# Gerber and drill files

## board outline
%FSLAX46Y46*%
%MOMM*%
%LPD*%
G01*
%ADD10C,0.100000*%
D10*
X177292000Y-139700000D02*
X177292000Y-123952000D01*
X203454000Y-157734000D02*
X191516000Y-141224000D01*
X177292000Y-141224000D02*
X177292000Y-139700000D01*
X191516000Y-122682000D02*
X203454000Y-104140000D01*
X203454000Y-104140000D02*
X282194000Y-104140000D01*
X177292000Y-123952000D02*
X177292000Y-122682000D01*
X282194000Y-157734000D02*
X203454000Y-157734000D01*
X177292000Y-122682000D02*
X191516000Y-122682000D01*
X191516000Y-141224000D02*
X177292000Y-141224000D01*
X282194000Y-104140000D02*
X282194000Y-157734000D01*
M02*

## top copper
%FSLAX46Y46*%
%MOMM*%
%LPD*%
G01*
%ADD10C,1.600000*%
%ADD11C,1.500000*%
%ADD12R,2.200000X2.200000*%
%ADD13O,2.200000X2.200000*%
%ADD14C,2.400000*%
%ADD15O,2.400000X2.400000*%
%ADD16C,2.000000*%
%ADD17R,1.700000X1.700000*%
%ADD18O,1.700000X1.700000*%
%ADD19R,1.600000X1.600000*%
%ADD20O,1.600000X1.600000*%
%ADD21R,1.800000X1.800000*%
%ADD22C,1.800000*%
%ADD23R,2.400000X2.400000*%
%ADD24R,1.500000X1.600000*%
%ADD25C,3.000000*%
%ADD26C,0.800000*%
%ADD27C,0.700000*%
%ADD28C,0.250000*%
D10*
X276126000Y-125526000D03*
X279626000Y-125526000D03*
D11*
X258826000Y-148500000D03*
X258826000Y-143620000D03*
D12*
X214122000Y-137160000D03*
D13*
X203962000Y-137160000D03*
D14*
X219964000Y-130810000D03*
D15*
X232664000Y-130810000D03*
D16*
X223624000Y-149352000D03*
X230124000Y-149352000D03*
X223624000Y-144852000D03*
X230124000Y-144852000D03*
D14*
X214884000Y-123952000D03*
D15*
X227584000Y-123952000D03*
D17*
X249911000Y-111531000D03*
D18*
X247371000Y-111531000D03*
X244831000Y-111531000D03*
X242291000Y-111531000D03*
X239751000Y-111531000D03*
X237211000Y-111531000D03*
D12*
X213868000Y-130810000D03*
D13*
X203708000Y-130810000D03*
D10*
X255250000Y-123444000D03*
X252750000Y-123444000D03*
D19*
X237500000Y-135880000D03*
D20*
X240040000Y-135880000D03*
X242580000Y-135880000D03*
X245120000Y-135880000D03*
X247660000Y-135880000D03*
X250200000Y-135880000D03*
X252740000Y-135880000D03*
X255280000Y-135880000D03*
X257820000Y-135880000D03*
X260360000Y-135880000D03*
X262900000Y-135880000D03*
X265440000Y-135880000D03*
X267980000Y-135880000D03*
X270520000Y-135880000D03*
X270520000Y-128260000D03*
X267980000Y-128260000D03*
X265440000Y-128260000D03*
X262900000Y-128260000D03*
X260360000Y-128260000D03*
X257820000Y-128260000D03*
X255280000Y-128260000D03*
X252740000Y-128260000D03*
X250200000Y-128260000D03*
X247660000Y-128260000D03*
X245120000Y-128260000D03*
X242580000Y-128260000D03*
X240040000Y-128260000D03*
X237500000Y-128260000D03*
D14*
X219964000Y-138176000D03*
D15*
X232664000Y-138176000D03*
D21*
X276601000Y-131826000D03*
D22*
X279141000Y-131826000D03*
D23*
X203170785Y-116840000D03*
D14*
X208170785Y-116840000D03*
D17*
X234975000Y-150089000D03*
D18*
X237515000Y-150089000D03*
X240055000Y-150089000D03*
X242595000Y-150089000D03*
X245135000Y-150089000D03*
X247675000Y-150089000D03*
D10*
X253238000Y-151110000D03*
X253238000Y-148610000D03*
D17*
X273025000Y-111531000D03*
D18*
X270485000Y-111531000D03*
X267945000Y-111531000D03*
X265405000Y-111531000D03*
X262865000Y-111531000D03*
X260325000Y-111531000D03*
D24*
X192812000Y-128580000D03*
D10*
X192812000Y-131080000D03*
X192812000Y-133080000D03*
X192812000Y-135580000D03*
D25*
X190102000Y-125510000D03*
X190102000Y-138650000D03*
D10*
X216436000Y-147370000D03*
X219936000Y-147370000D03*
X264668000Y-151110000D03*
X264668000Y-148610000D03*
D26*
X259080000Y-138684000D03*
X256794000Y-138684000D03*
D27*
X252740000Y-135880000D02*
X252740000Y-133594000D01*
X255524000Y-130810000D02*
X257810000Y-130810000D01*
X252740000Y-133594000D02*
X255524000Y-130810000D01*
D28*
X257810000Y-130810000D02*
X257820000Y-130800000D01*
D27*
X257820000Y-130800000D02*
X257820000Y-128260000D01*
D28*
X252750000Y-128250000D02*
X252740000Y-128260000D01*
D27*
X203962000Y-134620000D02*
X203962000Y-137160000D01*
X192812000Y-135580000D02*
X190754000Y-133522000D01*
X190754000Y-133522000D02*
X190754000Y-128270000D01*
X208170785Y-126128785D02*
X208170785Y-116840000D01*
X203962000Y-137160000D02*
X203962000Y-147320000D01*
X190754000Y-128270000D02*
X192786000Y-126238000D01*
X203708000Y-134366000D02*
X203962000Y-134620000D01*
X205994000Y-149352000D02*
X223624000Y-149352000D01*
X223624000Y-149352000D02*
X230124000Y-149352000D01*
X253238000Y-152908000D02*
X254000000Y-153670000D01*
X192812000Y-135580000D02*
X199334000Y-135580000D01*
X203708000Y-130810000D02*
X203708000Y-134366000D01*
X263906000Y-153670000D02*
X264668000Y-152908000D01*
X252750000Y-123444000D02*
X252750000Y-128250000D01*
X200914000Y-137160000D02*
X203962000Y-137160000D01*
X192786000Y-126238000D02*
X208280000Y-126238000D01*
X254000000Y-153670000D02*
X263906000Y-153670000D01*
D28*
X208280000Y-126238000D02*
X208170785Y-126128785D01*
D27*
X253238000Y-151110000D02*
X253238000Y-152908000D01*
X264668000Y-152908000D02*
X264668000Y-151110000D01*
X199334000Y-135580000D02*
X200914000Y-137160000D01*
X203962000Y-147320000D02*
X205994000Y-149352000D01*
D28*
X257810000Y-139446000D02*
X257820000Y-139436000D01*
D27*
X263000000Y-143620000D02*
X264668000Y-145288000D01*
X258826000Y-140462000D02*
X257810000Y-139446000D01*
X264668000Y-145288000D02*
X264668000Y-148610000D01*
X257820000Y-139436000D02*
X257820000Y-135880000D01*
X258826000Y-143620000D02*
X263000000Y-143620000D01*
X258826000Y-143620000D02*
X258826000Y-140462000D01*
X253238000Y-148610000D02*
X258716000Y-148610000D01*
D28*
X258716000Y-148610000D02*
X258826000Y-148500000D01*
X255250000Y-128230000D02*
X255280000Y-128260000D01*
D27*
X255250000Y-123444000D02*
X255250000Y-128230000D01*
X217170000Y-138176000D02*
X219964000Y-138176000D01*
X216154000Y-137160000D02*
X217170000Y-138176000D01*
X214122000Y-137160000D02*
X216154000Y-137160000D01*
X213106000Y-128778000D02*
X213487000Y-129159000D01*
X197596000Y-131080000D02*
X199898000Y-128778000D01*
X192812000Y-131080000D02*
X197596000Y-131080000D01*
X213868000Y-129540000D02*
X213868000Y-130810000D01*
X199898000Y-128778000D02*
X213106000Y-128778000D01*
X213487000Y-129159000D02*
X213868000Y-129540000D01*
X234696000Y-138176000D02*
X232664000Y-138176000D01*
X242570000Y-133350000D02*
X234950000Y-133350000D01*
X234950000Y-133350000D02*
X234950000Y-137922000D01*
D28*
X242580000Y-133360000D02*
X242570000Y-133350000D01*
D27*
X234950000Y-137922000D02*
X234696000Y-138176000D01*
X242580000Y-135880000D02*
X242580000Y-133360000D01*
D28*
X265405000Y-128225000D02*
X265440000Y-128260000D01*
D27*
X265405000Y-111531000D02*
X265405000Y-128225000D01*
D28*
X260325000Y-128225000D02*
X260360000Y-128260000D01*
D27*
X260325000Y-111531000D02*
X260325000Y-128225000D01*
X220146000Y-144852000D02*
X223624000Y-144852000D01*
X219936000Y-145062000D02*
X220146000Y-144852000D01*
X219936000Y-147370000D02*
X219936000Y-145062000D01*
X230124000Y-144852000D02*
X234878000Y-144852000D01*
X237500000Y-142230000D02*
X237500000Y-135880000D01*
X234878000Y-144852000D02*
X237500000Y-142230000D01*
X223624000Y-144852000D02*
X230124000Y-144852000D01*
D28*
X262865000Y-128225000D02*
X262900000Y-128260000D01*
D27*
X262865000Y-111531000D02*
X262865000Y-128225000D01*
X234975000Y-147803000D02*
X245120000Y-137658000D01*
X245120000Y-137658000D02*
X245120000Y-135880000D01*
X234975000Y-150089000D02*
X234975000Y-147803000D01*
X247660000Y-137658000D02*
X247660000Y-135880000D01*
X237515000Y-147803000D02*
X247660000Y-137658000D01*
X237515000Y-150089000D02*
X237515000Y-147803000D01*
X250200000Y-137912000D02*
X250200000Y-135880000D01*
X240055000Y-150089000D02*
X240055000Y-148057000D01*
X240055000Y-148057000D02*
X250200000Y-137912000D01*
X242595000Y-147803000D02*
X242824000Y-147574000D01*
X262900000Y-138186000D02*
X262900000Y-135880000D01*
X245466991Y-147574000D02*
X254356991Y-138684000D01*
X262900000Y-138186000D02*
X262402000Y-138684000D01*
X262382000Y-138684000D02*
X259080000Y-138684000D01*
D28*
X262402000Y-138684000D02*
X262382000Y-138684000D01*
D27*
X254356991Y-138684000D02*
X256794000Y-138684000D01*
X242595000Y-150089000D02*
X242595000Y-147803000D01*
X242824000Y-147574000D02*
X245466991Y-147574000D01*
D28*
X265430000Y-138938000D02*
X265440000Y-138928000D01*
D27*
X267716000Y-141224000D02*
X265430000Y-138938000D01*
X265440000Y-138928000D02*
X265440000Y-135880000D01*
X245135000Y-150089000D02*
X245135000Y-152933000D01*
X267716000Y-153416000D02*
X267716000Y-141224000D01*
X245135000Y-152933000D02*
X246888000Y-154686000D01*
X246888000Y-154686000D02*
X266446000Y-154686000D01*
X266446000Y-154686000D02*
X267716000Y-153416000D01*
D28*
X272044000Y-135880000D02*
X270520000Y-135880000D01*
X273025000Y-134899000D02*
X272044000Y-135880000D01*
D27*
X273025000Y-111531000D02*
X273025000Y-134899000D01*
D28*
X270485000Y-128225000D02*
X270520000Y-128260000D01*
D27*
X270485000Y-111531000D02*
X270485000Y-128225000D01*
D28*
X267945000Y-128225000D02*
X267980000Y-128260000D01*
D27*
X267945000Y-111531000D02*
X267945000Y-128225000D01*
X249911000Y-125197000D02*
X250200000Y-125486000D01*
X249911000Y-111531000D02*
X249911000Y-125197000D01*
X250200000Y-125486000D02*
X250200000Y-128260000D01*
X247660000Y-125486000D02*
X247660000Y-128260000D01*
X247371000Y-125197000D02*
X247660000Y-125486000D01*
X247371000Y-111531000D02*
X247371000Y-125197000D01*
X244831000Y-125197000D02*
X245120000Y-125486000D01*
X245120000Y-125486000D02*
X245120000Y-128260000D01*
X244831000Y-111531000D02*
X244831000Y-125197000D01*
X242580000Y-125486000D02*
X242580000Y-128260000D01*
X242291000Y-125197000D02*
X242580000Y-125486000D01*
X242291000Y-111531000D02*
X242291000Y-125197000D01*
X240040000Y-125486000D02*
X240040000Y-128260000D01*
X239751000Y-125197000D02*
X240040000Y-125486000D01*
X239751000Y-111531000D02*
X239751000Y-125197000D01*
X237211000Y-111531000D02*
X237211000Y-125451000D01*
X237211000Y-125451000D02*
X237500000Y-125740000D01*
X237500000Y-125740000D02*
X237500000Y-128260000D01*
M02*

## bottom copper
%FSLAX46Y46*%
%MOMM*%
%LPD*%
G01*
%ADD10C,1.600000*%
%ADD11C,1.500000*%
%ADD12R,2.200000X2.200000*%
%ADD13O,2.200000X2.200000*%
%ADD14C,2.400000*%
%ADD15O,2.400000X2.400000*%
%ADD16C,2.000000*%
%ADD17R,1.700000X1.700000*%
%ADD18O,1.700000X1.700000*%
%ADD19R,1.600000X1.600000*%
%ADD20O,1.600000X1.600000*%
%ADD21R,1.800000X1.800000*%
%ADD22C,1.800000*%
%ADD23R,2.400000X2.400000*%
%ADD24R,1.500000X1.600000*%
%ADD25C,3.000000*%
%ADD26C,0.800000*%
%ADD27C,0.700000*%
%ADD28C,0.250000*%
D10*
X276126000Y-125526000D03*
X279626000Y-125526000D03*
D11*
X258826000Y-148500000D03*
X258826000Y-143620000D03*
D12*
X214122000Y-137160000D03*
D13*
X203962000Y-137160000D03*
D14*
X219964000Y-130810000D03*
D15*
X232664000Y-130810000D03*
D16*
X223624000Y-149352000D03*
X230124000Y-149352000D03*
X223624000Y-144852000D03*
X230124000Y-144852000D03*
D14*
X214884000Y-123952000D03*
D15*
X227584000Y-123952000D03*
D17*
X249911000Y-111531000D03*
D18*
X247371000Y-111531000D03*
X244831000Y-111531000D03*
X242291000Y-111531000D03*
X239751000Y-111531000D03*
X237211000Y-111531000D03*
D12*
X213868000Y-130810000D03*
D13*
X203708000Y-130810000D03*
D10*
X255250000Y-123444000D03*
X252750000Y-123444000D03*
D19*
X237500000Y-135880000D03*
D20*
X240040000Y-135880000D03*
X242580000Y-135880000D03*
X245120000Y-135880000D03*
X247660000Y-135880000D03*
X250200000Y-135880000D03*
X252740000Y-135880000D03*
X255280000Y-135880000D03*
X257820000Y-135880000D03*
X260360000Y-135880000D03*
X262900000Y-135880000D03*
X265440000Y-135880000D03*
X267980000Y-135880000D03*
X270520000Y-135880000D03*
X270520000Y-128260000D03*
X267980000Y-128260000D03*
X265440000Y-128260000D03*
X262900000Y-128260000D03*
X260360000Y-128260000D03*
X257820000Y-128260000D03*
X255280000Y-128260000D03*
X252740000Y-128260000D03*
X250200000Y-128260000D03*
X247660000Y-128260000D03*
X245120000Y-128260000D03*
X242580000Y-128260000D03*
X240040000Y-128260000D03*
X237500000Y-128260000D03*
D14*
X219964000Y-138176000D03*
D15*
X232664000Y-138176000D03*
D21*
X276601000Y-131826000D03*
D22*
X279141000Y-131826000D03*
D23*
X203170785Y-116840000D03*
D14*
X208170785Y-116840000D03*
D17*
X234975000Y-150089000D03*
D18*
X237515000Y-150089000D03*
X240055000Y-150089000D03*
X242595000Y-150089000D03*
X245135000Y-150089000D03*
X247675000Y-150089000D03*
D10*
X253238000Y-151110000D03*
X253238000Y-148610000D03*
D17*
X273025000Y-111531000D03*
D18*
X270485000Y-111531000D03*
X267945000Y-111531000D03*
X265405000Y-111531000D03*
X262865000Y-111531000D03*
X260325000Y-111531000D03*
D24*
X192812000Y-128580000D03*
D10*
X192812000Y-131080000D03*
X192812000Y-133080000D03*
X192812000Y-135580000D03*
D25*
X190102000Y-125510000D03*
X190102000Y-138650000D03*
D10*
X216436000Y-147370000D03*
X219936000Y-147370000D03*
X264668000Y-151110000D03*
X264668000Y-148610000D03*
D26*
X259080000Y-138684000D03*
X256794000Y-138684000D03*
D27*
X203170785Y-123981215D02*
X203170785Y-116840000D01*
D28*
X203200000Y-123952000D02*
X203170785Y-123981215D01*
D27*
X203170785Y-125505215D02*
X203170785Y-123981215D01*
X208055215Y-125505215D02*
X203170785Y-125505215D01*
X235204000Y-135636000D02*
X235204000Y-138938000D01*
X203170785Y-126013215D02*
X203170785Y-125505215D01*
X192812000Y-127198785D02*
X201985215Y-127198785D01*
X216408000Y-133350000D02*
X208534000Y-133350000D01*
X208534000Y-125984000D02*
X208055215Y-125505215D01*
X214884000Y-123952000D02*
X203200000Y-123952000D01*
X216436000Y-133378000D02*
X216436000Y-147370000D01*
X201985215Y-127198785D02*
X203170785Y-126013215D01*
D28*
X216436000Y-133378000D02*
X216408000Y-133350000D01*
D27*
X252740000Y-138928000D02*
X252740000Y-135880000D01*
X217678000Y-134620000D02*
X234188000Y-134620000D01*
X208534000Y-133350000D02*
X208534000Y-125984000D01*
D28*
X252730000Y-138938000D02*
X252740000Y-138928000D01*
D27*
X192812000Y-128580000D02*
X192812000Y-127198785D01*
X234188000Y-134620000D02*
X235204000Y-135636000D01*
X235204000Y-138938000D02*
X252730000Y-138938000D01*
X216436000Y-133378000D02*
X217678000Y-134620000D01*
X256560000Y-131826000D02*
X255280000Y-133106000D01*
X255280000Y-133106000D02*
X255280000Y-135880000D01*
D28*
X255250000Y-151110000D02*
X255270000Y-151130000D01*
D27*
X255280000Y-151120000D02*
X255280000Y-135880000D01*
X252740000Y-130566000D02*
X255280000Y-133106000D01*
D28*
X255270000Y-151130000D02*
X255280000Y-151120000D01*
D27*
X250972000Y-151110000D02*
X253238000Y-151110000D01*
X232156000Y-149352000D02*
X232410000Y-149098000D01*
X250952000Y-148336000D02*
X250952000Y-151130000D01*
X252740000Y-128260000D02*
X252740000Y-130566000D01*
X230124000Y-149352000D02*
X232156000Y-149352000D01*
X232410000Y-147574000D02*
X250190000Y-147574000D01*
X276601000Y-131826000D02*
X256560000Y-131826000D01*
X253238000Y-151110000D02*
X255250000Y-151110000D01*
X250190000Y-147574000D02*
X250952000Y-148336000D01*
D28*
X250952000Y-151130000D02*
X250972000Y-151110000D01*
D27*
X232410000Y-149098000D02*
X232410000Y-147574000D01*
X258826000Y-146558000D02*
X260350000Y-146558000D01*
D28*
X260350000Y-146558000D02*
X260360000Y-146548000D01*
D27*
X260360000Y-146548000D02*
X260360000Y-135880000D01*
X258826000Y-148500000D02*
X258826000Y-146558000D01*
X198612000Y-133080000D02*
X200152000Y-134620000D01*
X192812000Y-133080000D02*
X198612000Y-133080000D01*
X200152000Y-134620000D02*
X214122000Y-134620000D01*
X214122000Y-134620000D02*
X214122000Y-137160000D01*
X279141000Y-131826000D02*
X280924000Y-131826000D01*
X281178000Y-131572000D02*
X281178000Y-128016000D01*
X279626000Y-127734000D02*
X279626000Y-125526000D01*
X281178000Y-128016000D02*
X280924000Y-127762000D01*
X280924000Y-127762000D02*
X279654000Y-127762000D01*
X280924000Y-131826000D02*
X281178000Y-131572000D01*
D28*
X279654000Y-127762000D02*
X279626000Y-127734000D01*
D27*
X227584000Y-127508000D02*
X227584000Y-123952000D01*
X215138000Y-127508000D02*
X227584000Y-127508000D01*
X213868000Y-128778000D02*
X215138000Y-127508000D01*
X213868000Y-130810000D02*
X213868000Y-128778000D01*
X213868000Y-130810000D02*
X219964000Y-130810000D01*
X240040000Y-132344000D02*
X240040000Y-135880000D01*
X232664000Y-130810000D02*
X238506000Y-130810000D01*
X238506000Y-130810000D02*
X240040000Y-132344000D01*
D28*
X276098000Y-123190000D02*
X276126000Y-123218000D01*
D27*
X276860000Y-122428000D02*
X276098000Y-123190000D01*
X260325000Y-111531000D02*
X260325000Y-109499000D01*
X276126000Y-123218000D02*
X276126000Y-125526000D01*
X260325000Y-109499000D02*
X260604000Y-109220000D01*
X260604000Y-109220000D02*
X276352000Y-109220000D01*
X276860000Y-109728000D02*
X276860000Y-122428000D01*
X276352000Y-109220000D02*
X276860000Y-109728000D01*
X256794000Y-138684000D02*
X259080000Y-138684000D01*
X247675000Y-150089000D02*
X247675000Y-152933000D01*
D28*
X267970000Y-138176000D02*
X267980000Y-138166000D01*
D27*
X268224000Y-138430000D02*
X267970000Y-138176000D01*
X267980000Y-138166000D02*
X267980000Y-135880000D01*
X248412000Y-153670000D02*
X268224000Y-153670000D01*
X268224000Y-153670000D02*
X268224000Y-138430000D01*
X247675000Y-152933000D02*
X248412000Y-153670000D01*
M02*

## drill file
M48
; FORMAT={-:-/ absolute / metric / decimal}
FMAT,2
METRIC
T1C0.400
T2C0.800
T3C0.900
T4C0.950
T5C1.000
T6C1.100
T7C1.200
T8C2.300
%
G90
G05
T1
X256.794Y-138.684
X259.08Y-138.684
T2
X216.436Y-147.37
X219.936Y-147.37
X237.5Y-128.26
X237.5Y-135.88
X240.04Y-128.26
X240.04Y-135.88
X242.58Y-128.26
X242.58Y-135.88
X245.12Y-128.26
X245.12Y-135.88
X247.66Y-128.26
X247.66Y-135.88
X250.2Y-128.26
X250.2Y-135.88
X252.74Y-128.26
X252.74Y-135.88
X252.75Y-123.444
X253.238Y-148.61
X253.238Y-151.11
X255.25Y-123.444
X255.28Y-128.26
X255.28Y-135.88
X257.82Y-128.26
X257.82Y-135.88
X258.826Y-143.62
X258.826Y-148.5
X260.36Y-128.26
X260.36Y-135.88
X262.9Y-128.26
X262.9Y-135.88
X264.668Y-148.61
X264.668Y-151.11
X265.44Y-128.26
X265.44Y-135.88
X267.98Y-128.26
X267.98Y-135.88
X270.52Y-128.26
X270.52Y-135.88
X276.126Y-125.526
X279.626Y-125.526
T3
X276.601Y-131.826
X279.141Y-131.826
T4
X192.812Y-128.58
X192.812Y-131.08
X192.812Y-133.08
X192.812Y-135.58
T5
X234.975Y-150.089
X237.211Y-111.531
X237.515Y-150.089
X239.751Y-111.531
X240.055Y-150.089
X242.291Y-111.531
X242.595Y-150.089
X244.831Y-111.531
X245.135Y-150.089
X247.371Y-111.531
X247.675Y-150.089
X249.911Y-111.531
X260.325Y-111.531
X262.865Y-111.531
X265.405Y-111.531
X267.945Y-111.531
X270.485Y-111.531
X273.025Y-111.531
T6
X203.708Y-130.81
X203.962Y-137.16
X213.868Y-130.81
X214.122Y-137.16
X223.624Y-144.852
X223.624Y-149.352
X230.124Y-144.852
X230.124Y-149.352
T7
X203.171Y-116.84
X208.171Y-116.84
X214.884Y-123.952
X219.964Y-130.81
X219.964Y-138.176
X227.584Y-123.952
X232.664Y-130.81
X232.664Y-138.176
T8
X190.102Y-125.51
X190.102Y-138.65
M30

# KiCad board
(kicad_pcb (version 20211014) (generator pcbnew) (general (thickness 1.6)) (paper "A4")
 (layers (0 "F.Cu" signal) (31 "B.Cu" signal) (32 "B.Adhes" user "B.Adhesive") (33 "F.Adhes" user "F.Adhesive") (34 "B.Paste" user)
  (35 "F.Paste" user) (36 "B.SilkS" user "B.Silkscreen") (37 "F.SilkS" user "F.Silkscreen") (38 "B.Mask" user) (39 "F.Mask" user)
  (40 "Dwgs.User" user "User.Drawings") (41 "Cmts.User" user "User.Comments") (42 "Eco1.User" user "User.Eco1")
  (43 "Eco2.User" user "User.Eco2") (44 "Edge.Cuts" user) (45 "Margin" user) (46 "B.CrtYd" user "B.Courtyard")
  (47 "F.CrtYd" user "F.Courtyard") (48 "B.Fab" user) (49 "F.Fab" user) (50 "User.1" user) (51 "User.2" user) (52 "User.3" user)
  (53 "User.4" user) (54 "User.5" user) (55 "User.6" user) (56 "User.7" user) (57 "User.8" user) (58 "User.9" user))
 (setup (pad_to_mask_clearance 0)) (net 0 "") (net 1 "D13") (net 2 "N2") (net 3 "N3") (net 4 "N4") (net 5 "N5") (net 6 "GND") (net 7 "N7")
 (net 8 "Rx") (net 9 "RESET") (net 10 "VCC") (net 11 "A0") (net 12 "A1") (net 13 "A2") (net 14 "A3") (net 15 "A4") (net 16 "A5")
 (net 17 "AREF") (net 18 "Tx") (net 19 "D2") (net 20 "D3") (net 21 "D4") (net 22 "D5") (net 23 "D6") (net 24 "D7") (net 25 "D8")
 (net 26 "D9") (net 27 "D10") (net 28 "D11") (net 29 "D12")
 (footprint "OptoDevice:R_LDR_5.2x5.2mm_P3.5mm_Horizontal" (layer "F.Cu") (at 276.126 125.526)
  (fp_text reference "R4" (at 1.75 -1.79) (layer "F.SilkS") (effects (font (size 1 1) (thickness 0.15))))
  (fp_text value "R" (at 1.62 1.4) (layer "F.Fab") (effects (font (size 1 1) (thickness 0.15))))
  (pad "1" thru_hole circle (at 0 0) (size 1.6 1.6) (drill 0.8) (layers *.Cu *.Mask) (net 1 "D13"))
  (pad "2" thru_hole circle (at 3.5 0) (size 1.6 1.6) (drill 0.8) (layers *.Cu *.Mask) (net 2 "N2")))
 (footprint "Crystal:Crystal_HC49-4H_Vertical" (layer "F.Cu") (at 258.826 148.5 90)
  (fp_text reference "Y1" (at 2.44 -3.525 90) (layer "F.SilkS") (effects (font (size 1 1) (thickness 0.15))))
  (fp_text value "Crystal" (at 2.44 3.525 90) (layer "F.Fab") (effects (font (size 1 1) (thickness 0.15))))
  (pad "1" thru_hole circle (at 0 0 90) (size 1.5 1.5) (drill 0.8) (layers *.Cu *.Mask) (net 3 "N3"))
  (pad "2" thru_hole circle (at 4.88 0 90) (size 1.5 1.5) (drill 0.8) (layers *.Cu *.Mask) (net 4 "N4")))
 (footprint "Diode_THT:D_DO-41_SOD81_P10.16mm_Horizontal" (layer "F.Cu") (at 214.122 137.16 180)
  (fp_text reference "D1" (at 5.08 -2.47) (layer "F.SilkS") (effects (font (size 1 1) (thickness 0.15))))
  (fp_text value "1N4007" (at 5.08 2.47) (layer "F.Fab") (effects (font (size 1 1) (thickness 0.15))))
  (pad "1" thru_hole rect (at 0 0 180) (size 2.2 2.2) (drill 1.1) (layers *.Cu *.Mask) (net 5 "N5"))
  (pad "2" thru_hole oval (at 10.16 0 180) (size 2.2 2.2) (drill 1.1) (layers *.Cu *.Mask) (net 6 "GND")))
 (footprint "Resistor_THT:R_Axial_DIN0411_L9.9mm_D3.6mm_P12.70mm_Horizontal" (layer "F.Cu") (at 219.964 130.81)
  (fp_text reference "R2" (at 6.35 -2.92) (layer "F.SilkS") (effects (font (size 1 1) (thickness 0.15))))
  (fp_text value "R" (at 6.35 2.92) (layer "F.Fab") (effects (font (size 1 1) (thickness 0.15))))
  (pad "1" thru_hole circle (at 0 0) (size 2.4 2.4) (drill 1.2) (layers *.Cu *.Mask) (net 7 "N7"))
  (pad "2" thru_hole oval (at 12.7 0) (size 2.4 2.4) (drill 1.2) (layers *.Cu *.Mask) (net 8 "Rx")))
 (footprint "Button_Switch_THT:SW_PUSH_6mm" (layer "F.Cu") (at 230.124 149.352 180)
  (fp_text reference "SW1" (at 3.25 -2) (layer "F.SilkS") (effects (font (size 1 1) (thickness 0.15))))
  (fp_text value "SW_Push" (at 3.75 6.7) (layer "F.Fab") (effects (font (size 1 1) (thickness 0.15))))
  (pad "1" thru_hole circle (at 6.5 0 270) (size 2 2) (drill 1.1) (layers *.Cu *.Mask) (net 6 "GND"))
  (pad "1" thru_hole circle (at 0 0 270) (size 2 2) (drill 1.1) (layers *.Cu *.Mask) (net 6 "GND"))
  (pad "2" thru_hole circle (at 6.5 4.5 270) (size 2 2) (drill 1.1) (layers *.Cu *.Mask) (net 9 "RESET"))
  (pad "2" thru_hole circle (at 0 4.5 270) (size 2 2) (drill 1.1) (layers *.Cu *.Mask) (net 9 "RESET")))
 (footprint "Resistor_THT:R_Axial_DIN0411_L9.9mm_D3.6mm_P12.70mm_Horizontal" (layer "F.Cu") (at 214.884 123.952)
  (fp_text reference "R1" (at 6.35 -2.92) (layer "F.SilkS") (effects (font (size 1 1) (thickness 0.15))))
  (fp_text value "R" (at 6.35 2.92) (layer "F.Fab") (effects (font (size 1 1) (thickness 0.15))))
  (pad "1" thru_hole circle (at 0 0) (size 2.4 2.4) (drill 1.2) (layers *.Cu *.Mask) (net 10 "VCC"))
  (pad "2" thru_hole oval (at 12.7 0) (size 2.4 2.4) (drill 1.2) (layers *.Cu *.Mask) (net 7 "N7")))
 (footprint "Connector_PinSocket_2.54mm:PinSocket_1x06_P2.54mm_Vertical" (layer "F.Cu") (at 249.911 111.531 -90)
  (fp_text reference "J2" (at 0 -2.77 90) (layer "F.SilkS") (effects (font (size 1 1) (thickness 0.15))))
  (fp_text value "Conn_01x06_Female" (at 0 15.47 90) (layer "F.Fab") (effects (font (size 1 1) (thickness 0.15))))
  (pad "1" thru_hole rect (at 0 0 270) (size 1.7 1.7) (drill 1) (layers *.Cu *.Mask) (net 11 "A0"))
  (pad "2" thru_hole oval (at 0 2.54 270) (size 1.7 1.7) (drill 1) (layers *.Cu *.Mask) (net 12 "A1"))
  (pad "3" thru_hole oval (at 0 5.08 270) (size 1.7 1.7) (drill 1) (layers *.Cu *.Mask) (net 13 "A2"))
  (pad "4" thru_hole oval (at 0 7.62 270) (size 1.7 1.7) (drill 1) (layers *.Cu *.Mask) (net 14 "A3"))
  (pad "5" thru_hole oval (at 0 10.16 270) (size 1.7 1.7) (drill 1) (layers *.Cu *.Mask) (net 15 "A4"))
  (pad "6" thru_hole oval (at 0 12.7 270) (size 1.7 1.7) (drill 1) (layers *.Cu *.Mask) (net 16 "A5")))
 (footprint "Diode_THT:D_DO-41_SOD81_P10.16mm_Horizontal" (layer "F.Cu") (at 213.868 130.81 180)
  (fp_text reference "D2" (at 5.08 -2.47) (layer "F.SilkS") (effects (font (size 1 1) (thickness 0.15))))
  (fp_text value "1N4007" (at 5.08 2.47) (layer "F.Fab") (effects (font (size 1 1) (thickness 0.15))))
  (pad "1" thru_hole rect (at 0 0 180) (size 2.2 2.2) (drill 1.1) (layers *.Cu *.Mask) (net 7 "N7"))
  (pad "2" thru_hole oval (at 10.16 0 180) (size 2.2 2.2) (drill 1.1) (layers *.Cu *.Mask) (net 6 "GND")))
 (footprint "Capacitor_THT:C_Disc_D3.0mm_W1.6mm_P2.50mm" (layer "F.Cu") (at 255.25 123.444 180)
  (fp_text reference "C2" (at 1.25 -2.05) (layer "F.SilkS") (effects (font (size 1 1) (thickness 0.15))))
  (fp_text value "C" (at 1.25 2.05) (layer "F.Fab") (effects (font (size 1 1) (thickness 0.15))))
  (pad "1" thru_hole circle (at 0 0 180) (size 1.6 1.6) (drill 0.8) (layers *.Cu *.Mask) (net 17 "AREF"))
  (pad "2" thru_hole circle (at 2.5 0 180) (size 1.6 1.6) (drill 0.8) (layers *.Cu *.Mask) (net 6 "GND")))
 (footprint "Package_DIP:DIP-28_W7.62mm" (layer "F.Cu") (at 237.5 135.88 90)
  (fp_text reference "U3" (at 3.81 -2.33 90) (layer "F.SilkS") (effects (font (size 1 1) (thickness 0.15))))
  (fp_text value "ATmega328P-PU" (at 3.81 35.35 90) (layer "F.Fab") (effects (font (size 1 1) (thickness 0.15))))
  (pad "1" thru_hole rect (at 0 0 90) (size 1.6 1.6) (drill 0.8) (layers *.Cu *.Mask) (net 9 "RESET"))
  (pad "2" thru_hole oval (at 0 2.54 90) (size 1.6 1.6) (drill 0.8) (layers *.Cu *.Mask) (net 8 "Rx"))
  (pad "3" thru_hole oval (at 0 5.08 90) (size 1.6 1.6) (drill 0.8) (layers *.Cu *.Mask) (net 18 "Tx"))
  (pad "4" thru_hole oval (at 0 7.62 90) (size 1.6 1.6) (drill 0.8) (layers *.Cu *.Mask) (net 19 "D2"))
  (pad "5" thru_hole oval (at 0 10.16 90) (size 1.6 1.6) (drill 0.8) (layers *.Cu *.Mask) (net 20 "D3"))
  (pad "6" thru_hole oval (at 0 12.7 90) (size 1.6 1.6) (drill 0.8) (layers *.Cu *.Mask) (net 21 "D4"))
  (pad "7" thru_hole oval (at 0 15.24 90) (size 1.6 1.6) (drill 0.8) (layers *.Cu *.Mask) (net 10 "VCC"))
  (pad "8" thru_hole oval (at 0 17.78 90) (size 1.6 1.6) (drill 0.8) (layers *.Cu *.Mask) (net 6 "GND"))
  (pad "9" thru_hole oval (at 0 20.32 90) (size 1.6 1.6) (drill 0.8) (layers *.Cu *.Mask) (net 4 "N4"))
  (pad "10" thru_hole oval (at 0 22.86 90) (size 1.6 1.6) (drill 0.8) (layers *.Cu *.Mask) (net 3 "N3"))
  (pad "11" thru_hole oval (at 0 25.4 90) (size 1.6 1.6) (drill 0.8) (layers *.Cu *.Mask) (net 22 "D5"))
  (pad "12" thru_hole oval (at 0 27.94 90) (size 1.6 1.6) (drill 0.8) (layers *.Cu *.Mask) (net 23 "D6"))
  (pad "13" thru_hole oval (at 0 30.48 90) (size 1.6 1.6) (drill 0.8) (layers *.Cu *.Mask) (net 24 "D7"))
  (pad "14" thru_hole oval (at 0 33.02 90) (size 1.6 1.6) (drill 0.8) (layers *.Cu *.Mask) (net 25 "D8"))
  (pad "15" thru_hole oval (at 7.62 33.02 90) (size 1.6 1.6) (drill 0.8) (layers *.Cu *.Mask) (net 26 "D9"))
  (pad "16" thru_hole oval (at 7.62 30.48 90) (size 1.6 1.6) (drill 0.8) (layers *.Cu *.Mask) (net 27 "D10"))
  (pad "17" thru_hole oval (at 7.62 27.94 90) (size 1.6 1.6) (drill 0.8) (layers *.Cu *.Mask) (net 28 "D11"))
  (pad "18" thru_hole oval (at 7.62 25.4 90) (size 1.6 1.6) (drill 0.8) (layers *.Cu *.Mask) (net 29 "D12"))
  (pad "19" thru_hole oval (at 7.62 22.86 90) (size 1.6 1.6) (drill 0.8) (layers *.Cu *.Mask) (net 1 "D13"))
  (pad "20" thru_hole oval (at 7.62 20.32 90) (size 1.6 1.6) (drill 0.8) (layers *.Cu *.Mask) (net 10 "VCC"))
  (pad "21" thru_hole oval (at 7.62 17.78 90) (size 1.6 1.6) (drill 0.8) (layers *.Cu *.Mask) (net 17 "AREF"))
  (pad "22" thru_hole oval (at 7.62 15.24 90) (size 1.6 1.6) (drill 0.8) (layers *.Cu *.Mask) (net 6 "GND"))
  (pad "23" thru_hole oval (at 7.62 12.7 90) (size 1.6 1.6) (drill 0.8) (layers *.Cu *.Mask) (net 11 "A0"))
  (pad "24" thru_hole oval (at 7.62 10.16 90) (size 1.6 1.6) (drill 0.8) (layers *.Cu *.Mask) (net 12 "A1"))
  (pad "25" thru_hole oval (at 7.62 7.62 90) (size 1.6 1.6) (drill 0.8) (layers *.Cu *.Mask) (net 13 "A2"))
  (pad "26" thru_hole oval (at 7.62 5.08 90) (size 1.6 1.6) (drill 0.8) (layers *.Cu *.Mask) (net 14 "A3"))
  (pad "27" thru_hole oval (at 7.62 2.54 90) (size 1.6 1.6) (drill 0.8) (layers *.Cu *.Mask) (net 15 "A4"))
  (pad "28" thru_hole oval (at 7.62 0 90) (size 1.6 1.6) (drill 0.8) (layers *.Cu *.Mask) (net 16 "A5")))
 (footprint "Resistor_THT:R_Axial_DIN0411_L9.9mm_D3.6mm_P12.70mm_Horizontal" (layer "F.Cu") (at 219.964 138.176)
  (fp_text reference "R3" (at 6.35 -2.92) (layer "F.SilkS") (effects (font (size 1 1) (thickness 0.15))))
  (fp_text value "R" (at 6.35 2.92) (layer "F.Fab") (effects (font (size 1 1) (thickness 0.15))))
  (pad "1" thru_hole circle (at 0 0) (size 2.4 2.4) (drill 1.2) (layers *.Cu *.Mask) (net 5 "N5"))
  (pad "2" thru_hole oval (at 12.7 0) (size 2.4 2.4) (drill 1.2) (layers *.Cu *.Mask) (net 18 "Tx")))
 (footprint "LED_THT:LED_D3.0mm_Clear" (layer "F.Cu") (at 276.601 131.826)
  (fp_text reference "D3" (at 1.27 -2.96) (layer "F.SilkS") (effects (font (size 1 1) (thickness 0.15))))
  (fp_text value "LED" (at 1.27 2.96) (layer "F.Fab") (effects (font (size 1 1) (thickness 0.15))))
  (pad "1" thru_hole rect (at 0 0) (size 1.8 1.8) (drill 0.9) (layers *.Cu *.Mask) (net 6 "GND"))
  (pad "2" thru_hole circle (at 2.54 0) (size 1.8 1.8) (drill 0.9) (layers *.Cu *.Mask) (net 2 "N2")))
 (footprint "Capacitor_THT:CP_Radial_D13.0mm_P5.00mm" (layer "F.Cu") (at 203.170785 116.84)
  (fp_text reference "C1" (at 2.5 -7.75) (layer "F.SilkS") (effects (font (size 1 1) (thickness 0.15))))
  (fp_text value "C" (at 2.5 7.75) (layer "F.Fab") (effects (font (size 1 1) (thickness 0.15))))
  (pad "1" thru_hole rect (at 0 0) (size 2.4 2.4) (drill 1.2) (layers *.Cu *.Mask) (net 10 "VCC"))
  (pad "2" thru_hole circle (at 5 0) (size 2.4 2.4) (drill 1.2) (layers *.Cu *.Mask) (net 6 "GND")))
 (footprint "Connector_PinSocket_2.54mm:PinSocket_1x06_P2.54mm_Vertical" (layer "F.Cu") (at 234.975 150.089 90)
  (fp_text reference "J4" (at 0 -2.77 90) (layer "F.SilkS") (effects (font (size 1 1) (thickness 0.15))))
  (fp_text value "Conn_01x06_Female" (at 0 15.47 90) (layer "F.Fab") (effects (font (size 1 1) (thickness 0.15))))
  (pad "1" thru_hole rect (at 0 0 90) (size 1.7 1.7) (drill 1) (layers *.Cu *.Mask) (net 19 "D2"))
  (pad "2" thru_hole oval (at 0 2.54 90) (size 1.7 1.7) (drill 1) (layers *.Cu *.Mask) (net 20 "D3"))
  (pad "3" thru_hole oval (at 0 5.08 90) (size 1.7 1.7) (drill 1) (layers *.Cu *.Mask) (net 21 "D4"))
  (pad "4" thru_hole oval (at 0 7.62 90) (size 1.7 1.7) (drill 1) (layers *.Cu *.Mask) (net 22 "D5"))
  (pad "5" thru_hole oval (at 0 10.16 90) (size 1.7 1.7) (drill 1) (layers *.Cu *.Mask) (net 23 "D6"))
  (pad "6" thru_hole oval (at 0 12.7 90) (size 1.7 1.7) (drill 1) (layers *.Cu *.Mask) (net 24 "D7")))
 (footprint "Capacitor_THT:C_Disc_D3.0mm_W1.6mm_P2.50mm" (layer "F.Cu") (at 253.238 151.11 90)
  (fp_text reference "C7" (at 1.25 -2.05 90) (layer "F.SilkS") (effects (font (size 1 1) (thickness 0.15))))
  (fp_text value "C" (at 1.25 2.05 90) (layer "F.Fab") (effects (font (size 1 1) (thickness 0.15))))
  (pad "1" thru_hole circle (at 0 0 90) (size 1.6 1.6) (drill 0.8) (layers *.Cu *.Mask) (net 6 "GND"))
  (pad "2" thru_hole circle (at 2.5 0 90) (size 1.6 1.6) (drill 0.8) (layers *.Cu *.Mask) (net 3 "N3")))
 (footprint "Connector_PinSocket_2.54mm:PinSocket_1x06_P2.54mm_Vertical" (layer "F.Cu") (at 273.025 111.531 -90)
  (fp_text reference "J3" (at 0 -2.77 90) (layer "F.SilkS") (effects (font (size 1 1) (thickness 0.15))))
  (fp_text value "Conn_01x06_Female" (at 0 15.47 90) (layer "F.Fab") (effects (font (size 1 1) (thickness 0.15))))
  (pad "1" thru_hole rect (at 0 0 270) (size 1.7 1.7) (drill 1) (layers *.Cu *.Mask) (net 25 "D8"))
  (pad "2" thru_hole oval (at 0 2.54 270) (size 1.7 1.7) (drill 1) (layers *.Cu *.Mask) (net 26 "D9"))
  (pad "3" thru_hole oval (at 0 5.08 270) (size 1.7 1.7) (drill 1) (layers *.Cu *.Mask) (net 27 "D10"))
  (pad "4" thru_hole oval (at 0 7.62 270) (size 1.7 1.7) (drill 1) (layers *.Cu *.Mask) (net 28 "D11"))
  (pad "5" thru_hole oval (at 0 10.16 270) (size 1.7 1.7) (drill 1) (layers *.Cu *.Mask) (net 29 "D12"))
  (pad "6" thru_hole oval (at 0 12.7 270) (size 1.7 1.7) (drill 1) (layers *.Cu *.Mask) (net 1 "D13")))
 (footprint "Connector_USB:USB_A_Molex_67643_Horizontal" (layer "F.Cu") (at 192.812 128.58 -90)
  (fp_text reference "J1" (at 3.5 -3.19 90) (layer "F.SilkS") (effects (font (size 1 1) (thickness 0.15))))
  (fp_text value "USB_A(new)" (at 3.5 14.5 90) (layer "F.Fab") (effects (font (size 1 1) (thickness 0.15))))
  (pad "1" thru_hole rect (at 0 0 270) (size 1.6 1.5) (drill 0.95) (layers *.Cu *.Mask) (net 10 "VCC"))
  (pad "2" thru_hole circle (at 2.5 0 270) (size 1.6 1.6) (drill 0.95) (layers *.Cu *.Mask) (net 7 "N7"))
  (pad "3" thru_hole circle (at 4.5 0 270) (size 1.6 1.6) (drill 0.95) (layers *.Cu *.Mask) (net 5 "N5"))
  (pad "4" thru_hole circle (at 7 0 270) (size 1.6 1.6) (drill 0.95) (layers *.Cu *.Mask) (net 6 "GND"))
  (pad "5" thru_hole circle (at -3.07 2.71 270) (size 3 3) (drill 2.3) (layers *.Cu *.Mask))
  (pad "5" thru_hole circle (at 10.07 2.71 270) (size 3 3) (drill 2.3) (layers *.Cu *.Mask)))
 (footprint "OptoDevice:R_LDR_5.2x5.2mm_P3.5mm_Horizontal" (layer "F.Cu") (at 216.436 147.37)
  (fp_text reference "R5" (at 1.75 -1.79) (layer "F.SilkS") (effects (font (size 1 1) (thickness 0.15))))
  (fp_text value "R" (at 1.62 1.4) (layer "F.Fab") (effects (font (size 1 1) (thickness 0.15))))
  (pad "1" thru_hole circle (at 0 0) (size 1.6 1.6) (drill 0.8) (layers *.Cu *.Mask) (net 10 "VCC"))
  (pad "2" thru_hole circle (at 3.5 0) (size 1.6 1.6) (drill 0.8) (layers *.Cu *.Mask) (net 9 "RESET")))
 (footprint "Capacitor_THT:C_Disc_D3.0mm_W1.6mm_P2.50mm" (layer "F.Cu") (at 264.668 151.11 90)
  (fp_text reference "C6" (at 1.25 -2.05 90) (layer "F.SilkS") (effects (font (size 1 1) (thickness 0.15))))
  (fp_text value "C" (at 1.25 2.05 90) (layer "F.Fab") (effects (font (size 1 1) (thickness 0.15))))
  (pad "1" thru_hole circle (at 0 0 90) (size 1.6 1.6) (drill 0.8) (layers *.Cu *.Mask) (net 6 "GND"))
  (pad "2" thru_hole circle (at 2.5 0 90) (size 1.6 1.6) (drill 0.8) (layers *.Cu *.Mask) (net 4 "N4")))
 (gr_line (start 177.292 139.7) (end 177.292 123.952) (layer "Edge.Cuts") (width 0.1))
 (gr_line (start 203.454 157.734) (end 191.516 141.224) (layer "Edge.Cuts") (width 0.1))
 (gr_line (start 177.292 141.224) (end 177.292 139.7) (layer "Edge.Cuts") (width 0.1))
 (gr_line (start 191.516 122.682) (end 203.454 104.14) (layer "Edge.Cuts") (width 0.1))
 (gr_line (start 203.454 104.14) (end 282.194 104.14) (layer "Edge.Cuts") (width 0.1))
 (gr_line (start 177.292 123.952) (end 177.292 122.682) (layer "Edge.Cuts") (width 0.1))
 (gr_line (start 282.194 157.734) (end 203.454 157.734) (layer "Edge.Cuts") (width 0.1))
 (gr_line (start 177.292 122.682) (end 191.516 122.682) (layer "Edge.Cuts") (width 0.1))
 (gr_line (start 191.516 141.224) (end 177.292 141.224) (layer "Edge.Cuts") (width 0.1))
 (gr_line (start 282.194 104.14) (end 282.194 157.734) (layer "Edge.Cuts") (width 0.1))
 (segment (start 252.74 135.88) (end 252.74 133.594) (width 0.7) (layer "F.Cu") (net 10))
 (segment (start 255.524 130.81) (end 257.81 130.81) (width 0.7) (layer "F.Cu") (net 10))
 (segment (start 252.74 133.594) (end 255.524 130.81) (width 0.7) (layer "F.Cu") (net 10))
 (segment (start 257.81 130.81) (end 257.82 130.8) (width 0.25) (layer "F.Cu") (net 10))
 (segment (start 257.82 130.8) (end 257.82 128.26) (width 0.7) (layer "F.Cu") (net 10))
 (segment (start 203.170785 123.981215) (end 203.170785 116.84) (width 0.7) (layer "B.Cu") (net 10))
 (segment (start 203.2 123.952) (end 203.170785 123.981215) (width 0.25) (layer "B.Cu") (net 10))
 (segment (start 203.170785 125.505215) (end 203.170785 123.981215) (width 0.7) (layer "B.Cu") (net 10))
 (segment (start 208.055215 125.505215) (end 203.170785 125.505215) (width 0.7) (layer "B.Cu") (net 10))
 (segment (start 235.204 135.636) (end 235.204 138.938) (width 0.7) (layer "B.Cu") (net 10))
 (segment (start 203.170785 126.013215) (end 203.170785 125.505215) (width 0.7) (layer "B.Cu") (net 10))
 (segment (start 192.812 127.198785) (end 201.985215 127.198785) (width 0.7) (layer "B.Cu") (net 10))
 (segment (start 216.408 133.35) (end 208.534 133.35) (width 0.7) (layer "B.Cu") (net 10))
 (segment (start 208.534 125.984) (end 208.055215 125.505215) (width 0.7) (layer "B.Cu") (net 10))
 (segment (start 214.884 123.952) (end 203.2 123.952) (width 0.7) (layer "B.Cu") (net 10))
 (segment (start 216.436 133.378) (end 216.436 147.37) (width 0.7) (layer "B.Cu") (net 10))
 (segment (start 201.985215 127.198785) (end 203.170785 126.013215) (width 0.7) (layer "B.Cu") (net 10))
 (segment (start 216.436 133.378) (end 216.408 133.35) (width 0.25) (layer "B.Cu") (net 10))
 (segment (start 252.74 138.928) (end 252.74 135.88) (width 0.7) (layer "B.Cu") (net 10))
 (segment (start 217.678 134.62) (end 234.188 134.62) (width 0.7) (layer "B.Cu") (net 10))
 (segment (start 208.534 133.35) (end 208.534 125.984) (width 0.7) (layer "B.Cu") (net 10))
 (segment (start 252.73 138.938) (end 252.74 138.928) (width 0.25) (layer "B.Cu") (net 10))
 (segment (start 192.812 128.58) (end 192.812 127.198785) (width 0.7) (layer "B.Cu") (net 10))
 (segment (start 234.188 134.62) (end 235.204 135.636) (width 0.7) (layer "B.Cu") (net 10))
 (segment (start 235.204 138.938) (end 252.73 138.938) (width 0.7) (layer "B.Cu") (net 10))
 (segment (start 216.436 133.378) (end 217.678 134.62) (width 0.7) (layer "B.Cu") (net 10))
 (segment (start 252.75 128.25) (end 252.74 128.26) (width 0.25) (layer "F.Cu") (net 6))
 (segment (start 203.962 134.62) (end 203.962 137.16) (width 0.7) (layer "F.Cu") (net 6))
 (segment (start 192.812 135.58) (end 190.754 133.522) (width 0.7) (layer "F.Cu") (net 6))
 (segment (start 190.754 133.522) (end 190.754 128.27) (width 0.7) (layer "F.Cu") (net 6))
 (segment (start 208.170785 126.128785) (end 208.170785 116.84) (width 0.7) (layer "F.Cu") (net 6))
 (segment (start 203.962 137.16) (end 203.962 147.32) (width 0.7) (layer "F.Cu") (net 6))
 (segment (start 190.754 128.27) (end 192.786 126.238) (width 0.7) (layer "F.Cu") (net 6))
 (segment (start 203.708 134.366) (end 203.962 134.62) (width 0.7) (layer "F.Cu") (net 6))
 (segment (start 205.994 149.352) (end 223.624 149.352) (width 0.7) (layer "F.Cu") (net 6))
 (segment (start 223.624 149.352) (end 230.124 149.352) (width 0.7) (layer "F.Cu") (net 6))
 (segment (start 253.238 152.908) (end 254 153.67) (width 0.7) (layer "F.Cu") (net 6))
 (segment (start 192.812 135.58) (end 199.334 135.58) (width 0.7) (layer "F.Cu") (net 6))
 (segment (start 203.708 130.81) (end 203.708 134.366) (width 0.7) (layer "F.Cu") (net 6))
 (segment (start 263.906 153.67) (end 264.668 152.908) (width 0.7) (layer "F.Cu") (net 6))
 (segment (start 252.75 123.444) (end 252.75 128.25) (width 0.7) (layer "F.Cu") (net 6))
 (segment (start 200.914 137.16) (end 203.962 137.16) (width 0.7) (layer "F.Cu") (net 6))
 (segment (start 192.786 126.238) (end 208.28 126.238) (width 0.7) (layer "F.Cu") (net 6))
 (segment (start 254 153.67) (end 263.906 153.67) (width 0.7) (layer "F.Cu") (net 6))
 (segment (start 208.28 126.238) (end 208.170785 126.128785) (width 0.25) (layer "F.Cu") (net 6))
 (segment (start 253.238 151.11) (end 253.238 152.908) (width 0.7) (layer "F.Cu") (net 6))
 (segment (start 264.668 152.908) (end 264.668 151.11) (width 0.7) (layer "F.Cu") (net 6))
 (segment (start 199.334 135.58) (end 200.914 137.16) (width 0.7) (layer "F.Cu") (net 6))
 (segment (start 203.962 147.32) (end 205.994 149.352) (width 0.7) (layer "F.Cu") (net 6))
 (segment (start 256.56 131.826) (end 255.28 133.106) (width 0.7) (layer "B.Cu") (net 6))
 (segment (start 255.28 133.106) (end 255.28 135.88) (width 0.7) (layer "B.Cu") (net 6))
 (segment (start 255.25 151.11) (end 255.27 151.13) (width 0.25) (layer "B.Cu") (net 6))
 (segment (start 255.28 151.12) (end 255.28 135.88) (width 0.7) (layer "B.Cu") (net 6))
 (segment (start 252.74 130.566) (end 255.28 133.106) (width 0.7) (layer "B.Cu") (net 6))
 (segment (start 255.27 151.13) (end 255.28 151.12) (width 0.25) (layer "B.Cu") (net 6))
 (segment (start 250.972 151.11) (end 253.238 151.11) (width 0.7) (layer "B.Cu") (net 6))
 (segment (start 232.156 149.352) (end 232.41 149.098) (width 0.7) (layer "B.Cu") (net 6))
 (segment (start 250.952 148.336) (end 250.952 151.13) (width 0.7) (layer "B.Cu") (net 6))
 (segment (start 252.74 128.26) (end 252.74 130.566) (width 0.7) (layer "B.Cu") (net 6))
 (segment (start 230.124 149.352) (end 232.156 149.352) (width 0.7) (layer "B.Cu") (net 6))
 (segment (start 232.41 147.574) (end 250.19 147.574) (width 0.7) (layer "B.Cu") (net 6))
 (segment (start 276.601 131.826) (end 256.56 131.826) (width 0.7) (layer "B.Cu") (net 6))
 (segment (start 253.238 151.11) (end 255.25 151.11) (width 0.7) (layer "B.Cu") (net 6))
 (segment (start 250.19 147.574) (end 250.952 148.336) (width 0.7) (layer "B.Cu") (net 6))
 (segment (start 250.952 151.13) (end 250.972 151.11) (width 0.25) (layer "B.Cu") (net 6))
 (segment (start 232.41 149.098) (end 232.41 147.574) (width 0.7) (layer "B.Cu") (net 6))
 (segment (start 257.81 139.446) (end 257.82 139.436) (width 0.25) (layer "F.Cu") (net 4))
 (segment (start 263 143.62) (end 264.668 145.288) (width 0.7) (layer "F.Cu") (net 4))
 (segment (start 258.826 140.462) (end 257.81 139.446) (width 0.7) (layer "F.Cu") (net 4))
 (segment (start 264.668 145.288) (end 264.668 148.61) (width 0.7) (layer "F.Cu") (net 4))
 (segment (start 257.82 139.436) (end 257.82 135.88) (width 0.7) (layer "F.Cu") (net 4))
 (segment (start 258.826 143.62) (end 263 143.62) (width 0.7) (layer "F.Cu") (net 4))
 (segment (start 258.826 143.62) (end 258.826 140.462) (width 0.7) (layer "F.Cu") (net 4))
 (segment (start 253.238 148.61) (end 258.716 148.61) (width 0.7) (layer "F.Cu") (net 3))
 (segment (start 258.716 148.61) (end 258.826 148.5) (width 0.25) (layer "F.Cu") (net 3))
 (segment (start 258.826 146.558) (end 260.35 146.558) (width 0.7) (layer "B.Cu") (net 3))
 (segment (start 260.35 146.558) (end 260.36 146.548) (width 0.25) (layer "B.Cu") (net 3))
 (segment (start 260.36 146.548) (end 260.36 135.88) (width 0.7) (layer "B.Cu") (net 3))
 (segment (start 258.826 148.5) (end 258.826 146.558) (width 0.7) (layer "B.Cu") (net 3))
 (segment (start 255.25 128.23) (end 255.28 128.26) (width 0.25) (layer "F.Cu") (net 17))
 (segment (start 255.25 123.444) (end 255.25 128.23) (width 0.7) (layer "F.Cu") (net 17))
 (segment (start 217.17 138.176) (end 219.964 138.176) (width 0.7) (layer "F.Cu") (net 5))
 (segment (start 216.154 137.16) (end 217.17 138.176) (width 0.7) (layer "F.Cu") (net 5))
 (segment (start 214.122 137.16) (end 216.154 137.16) (width 0.7) (layer "F.Cu") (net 5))
 (segment (start 198.612 133.08) (end 200.152 134.62) (width 0.7) (layer "B.Cu") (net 5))
 (segment (start 192.812 133.08) (end 198.612 133.08) (width 0.7) (layer "B.Cu") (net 5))
 (segment (start 200.152 134.62) (end 214.122 134.62) (width 0.7) (layer "B.Cu") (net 5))
 (segment (start 214.122 134.62) (end 214.122 137.16) (width 0.7) (layer "B.Cu") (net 5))
 (segment (start 279.141 131.826) (end 280.924 131.826) (width 0.7) (layer "B.Cu") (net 2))
 (segment (start 281.178 131.572) (end 281.178 128.016) (width 0.7) (layer "B.Cu") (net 2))
 (segment (start 279.626 127.734) (end 279.626 125.526) (width 0.7) (layer "B.Cu") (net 2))
 (segment (start 281.178 128.016) (end 280.924 127.762) (width 0.7) (layer "B.Cu") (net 2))
 (segment (start 280.924 127.762) (end 279.654 127.762) (width 0.7) (layer "B.Cu") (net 2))
 (segment (start 280.924 131.826) (end 281.178 131.572) (width 0.7) (layer "B.Cu") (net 2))
 (segment (start 279.654 127.762) (end 279.626 127.734) (width 0.25) (layer "B.Cu") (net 2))
 (segment (start 213.106 128.778) (end 213.487 129.159) (width 0.7) (layer "F.Cu") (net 7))
 (segment (start 197.596 131.08) (end 199.898 128.778) (width 0.7) (layer "F.Cu") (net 7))
 (segment (start 192.812 131.08) (end 197.596 131.08) (width 0.7) (layer "F.Cu") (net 7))
 (segment (start 213.868 129.54) (end 213.868 130.81) (width 0.7) (layer "F.Cu") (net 7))
 (segment (start 199.898 128.778) (end 213.106 128.778) (width 0.7) (layer "F.Cu") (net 7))
 (segment (start 213.487 129.159) (end 213.868 129.54) (width 0.7) (layer "F.Cu") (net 7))
 (segment (start 227.584 127.508) (end 227.584 123.952) (width 0.7) (layer "B.Cu") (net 7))
 (segment (start 215.138 127.508) (end 227.584 127.508) (width 0.7) (layer "B.Cu") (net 7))
 (segment (start 213.868 128.778) (end 215.138 127.508) (width 0.7) (layer "B.Cu") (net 7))
 (segment (start 213.868 130.81) (end 213.868 128.778) (width 0.7) (layer "B.Cu") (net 7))
 (segment (start 213.868 130.81) (end 219.964 130.81) (width 0.7) (layer "B.Cu") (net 7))
 (segment (start 240.04 132.344) (end 240.04 135.88) (width 0.7) (layer "B.Cu") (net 8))
 (segment (start 232.664 130.81) (end 238.506 130.81) (width 0.7) (layer "B.Cu") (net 8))
 (segment (start 238.506 130.81) (end 240.04 132.344) (width 0.7) (layer "B.Cu") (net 8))
 (segment (start 234.696 138.176) (end 232.664 138.176) (width 0.7) (layer "F.Cu") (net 18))
 (segment (start 242.57 133.35) (end 234.95 133.35) (width 0.7) (layer "F.Cu") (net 18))
 (segment (start 234.95 133.35) (end 234.95 137.922) (width 0.7) (layer "F.Cu") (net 18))
 (segment (start 242.58 133.36) (end 242.57 133.35) (width 0.25) (layer "F.Cu") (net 18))
 (segment (start 234.95 137.922) (end 234.696 138.176) (width 0.7) (layer "F.Cu") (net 18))
 (segment (start 242.58 135.88) (end 242.58 133.36) (width 0.7) (layer "F.Cu") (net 18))
 (segment (start 265.405 128.225) (end 265.44 128.26) (width 0.25) (layer "F.Cu") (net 28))
 (segment (start 265.405 111.531) (end 265.405 128.225) (width 0.7) (layer "F.Cu") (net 28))
 (segment (start 260.325 128.225) (end 260.36 128.26) (width 0.25) (layer "F.Cu") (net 1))
 (segment (start 260.325 111.531) (end 260.325 128.225) (width 0.7) (layer "F.Cu") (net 1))
 (segment (start 276.098 123.19) (end 276.126 123.218) (width 0.25) (layer "B.Cu") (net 1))
 (segment (start 276.86 122.428) (end 276.098 123.19) (width 0.7) (layer "B.Cu") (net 1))
 (segment (start 260.325 111.531) (end 260.325 109.499) (width 0.7) (layer "B.Cu") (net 1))
 (segment (start 276.126 123.218) (end 276.126 125.526) (width 0.7) (layer "B.Cu") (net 1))
 (segment (start 260.325 109.499) (end 260.604 109.22) (width 0.7) (layer "B.Cu") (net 1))
 (segment (start 260.604 109.22) (end 276.352 109.22) (width 0.7) (layer "B.Cu") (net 1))
 (segment (start 276.86 109.728) (end 276.86 122.428) (width 0.7) (layer "B.Cu") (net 1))
 (segment (start 276.352 109.22) (end 276.86 109.728) (width 0.7) (layer "B.Cu") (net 1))
 (segment (start 220.146 144.852) (end 223.624 144.852) (width 0.7) (layer "F.Cu") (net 9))
 (segment (start 219.936 145.062) (end 220.146 144.852) (width 0.7) (layer "F.Cu") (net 9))
 (segment (start 219.936 147.37) (end 219.936 145.062) (width 0.7) (layer "F.Cu") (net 9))
 (segment (start 230.124 144.852) (end 234.878 144.852) (width 0.7) (layer "F.Cu") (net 9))
 (segment (start 237.5 142.23) (end 237.5 135.88) (width 0.7) (layer "F.Cu") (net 9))
 (segment (start 234.878 144.852) (end 237.5 142.23) (width 0.7) (layer "F.Cu") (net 9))
 (segment (start 223.624 144.852) (end 230.124 144.852) (width 0.7) (layer "F.Cu") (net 9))
 (segment (start 262.865 128.225) (end 262.9 128.26) (width 0.25) (layer "F.Cu") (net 29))
 (segment (start 262.865 111.531) (end 262.865 128.225) (width 0.7) (layer "F.Cu") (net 29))
 (segment (start 234.975 147.803) (end 245.12 137.658) (width 0.7) (layer "F.Cu") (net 19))
 (segment (start 245.12 137.658) (end 245.12 135.88) (width 0.7) (layer "F.Cu") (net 19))
 (segment (start 234.975 150.089) (end 234.975 147.803) (width 0.7) (layer "F.Cu") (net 19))
 (segment (start 247.66 137.658) (end 247.66 135.88) (width 0.7) (layer "F.Cu") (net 20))
 (segment (start 237.515 147.803) (end 247.66 137.658) (width 0.7) (layer "F.Cu") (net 20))
 (segment (start 237.515 150.089) (end 237.515 147.803) (width 0.7) (layer "F.Cu") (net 20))
 (segment (start 250.2 137.912) (end 250.2 135.88) (width 0.7) (layer "F.Cu") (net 21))
 (segment (start 240.055 150.089) (end 240.055 148.057) (width 0.7) (layer "F.Cu") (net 21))
 (segment (start 240.055 148.057) (end 250.2 137.912) (width 0.7) (layer "F.Cu") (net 21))
 (segment (start 242.595 147.803) (end 242.824 147.574) (width 0.7) (layer "F.Cu") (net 22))
 (segment (start 262.9 138.186) (end 262.9 135.88) (width 0.7) (layer "F.Cu") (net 22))
 (segment (start 245.466991 147.574) (end 254.356991 138.684) (width 0.7) (layer "F.Cu") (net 22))
 (segment (start 262.9 138.186) (end 262.402 138.684) (width 0.7) (layer "F.Cu") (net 22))
 (segment (start 262.382 138.684) (end 259.08 138.684) (width 0.7) (layer "F.Cu") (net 22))
 (segment (start 262.402 138.684) (end 262.382 138.684) (width 0.25) (layer "F.Cu") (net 22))
 (segment (start 254.356991 138.684) (end 256.794 138.684) (width 0.7) (layer "F.Cu") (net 22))
 (segment (start 242.595 150.089) (end 242.595 147.803) (width 0.7) (layer "F.Cu") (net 22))
 (segment (start 242.824 147.574) (end 245.466991 147.574) (width 0.7) (layer "F.Cu") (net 22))
 (via (at 259.08 138.684) (size 0.8) (drill 0.4) (layers "F.Cu" "B.Cu") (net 22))
 (via (at 256.794 138.684) (size 0.8) (drill 0.4) (layers "F.Cu" "B.Cu") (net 22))
 (segment (start 256.794 138.684) (end 259.08 138.684) (width 0.7) (layer "B.Cu") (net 22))
 (segment (start 265.43 138.938) (end 265.44 138.928) (width 0.25) (layer "F.Cu") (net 23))
 (segment (start 267.716 141.224) (end 265.43 138.938) (width 0.7) (layer "F.Cu") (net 23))
 (segment (start 265.44 138.928) (end 265.44 135.88) (width 0.7) (layer "F.Cu") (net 23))
 (segment (start 245.135 150.089) (end 245.135 152.933) (width 0.7) (layer "F.Cu") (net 23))
 (segment (start 267.716 153.416) (end 267.716 141.224) (width 0.7) (layer "F.Cu") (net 23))
 (segment (start 245.135 152.933) (end 246.888 154.686) (width 0.7) (layer "F.Cu") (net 23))
 (segment (start 246.888 154.686) (end 266.446 154.686) (width 0.7) (layer "F.Cu") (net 23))
 (segment (start 266.446 154.686) (end 267.716 153.416) (width 0.7) (layer "F.Cu") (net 23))
 (segment (start 247.675 150.089) (end 247.675 152.933) (width 0.7) (layer "B.Cu") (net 24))
 (segment (start 267.97 138.176) (end 267.98 138.166) (width 0.25) (layer "B.Cu") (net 24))
 (segment (start 268.224 138.43) (end 267.97 138.176) (width 0.7) (layer "B.Cu") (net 24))
 (segment (start 267.98 138.166) (end 267.98 135.88) (width 0.7) (layer "B.Cu") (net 24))
 (segment (start 248.412 153.67) (end 268.224 153.67) (width 0.7) (layer "B.Cu") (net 24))
 (segment (start 268.224 153.67) (end 268.224 138.43) (width 0.7) (layer "B.Cu") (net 24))
 (segment (start 247.675 152.933) (end 248.412 153.67) (width 0.7) (layer "B.Cu") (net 24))
 (segment (start 272.044 135.88) (end 270.52 135.88) (width 0.25) (layer "F.Cu") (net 25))
 (segment (start 273.025 134.899) (end 272.044 135.88) (width 0.25) (layer "F.Cu") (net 25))
 (segment (start 273.025 111.531) (end 273.025 134.899) (width 0.7) (layer "F.Cu") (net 25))
 (segment (start 270.485 128.225) (end 270.52 128.26) (width 0.25) (layer "F.Cu") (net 26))
 (segment (start 270.485 111.531) (end 270.485 128.225) (width 0.7) (layer "F.Cu") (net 26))
 (segment (start 267.945 128.225) (end 267.98 128.26) (width 0.25) (layer "F.Cu") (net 27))
 (segment (start 267.945 111.531) (end 267.945 128.225) (width 0.7) (layer "F.Cu") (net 27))
 (segment (start 249.911 125.197) (end 250.2 125.486) (width 0.7) (layer "F.Cu") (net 11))
 (segment (start 249.911 111.531) (end 249.911 125.197) (width 0.7) (layer "F.Cu") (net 11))
 (segment (start 250.2 125.486) (end 250.2 128.26) (width 0.7) (layer "F.Cu") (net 11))
 (segment (start 247.66 125.486) (end 247.66 128.26) (width 0.7) (layer "F.Cu") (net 12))
 (segment (start 247.371 125.197) (end 247.66 125.486) (width 0.7) (layer "F.Cu") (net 12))
 (segment (start 247.371 111.531) (end 247.371 125.197) (width 0.7) (layer "F.Cu") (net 12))
 (segment (start 244.831 125.197) (end 245.12 125.486) (width 0.7) (layer "F.Cu") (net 13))
 (segment (start 245.12 125.486) (end 245.12 128.26) (width 0.7) (layer "F.Cu") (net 13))
 (segment (start 244.831 111.531) (end 244.831 125.197) (width 0.7) (layer "F.Cu") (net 13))
 (segment (start 242.58 125.486) (end 242.58 128.26) (width 0.7) (layer "F.Cu") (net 14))
 (segment (start 242.291 125.197) (end 242.58 125.486) (width 0.7) (layer "F.Cu") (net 14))
 (segment (start 242.291 111.531) (end 242.291 125.197) (width 0.7) (layer "F.Cu") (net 14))
 (segment (start 240.04 125.486) (end 240.04 128.26) (width 0.7) (layer "F.Cu") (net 15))
 (segment (start 239.751 125.197) (end 240.04 125.486) (width 0.7) (layer "F.Cu") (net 15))
 (segment (start 239.751 111.531) (end 239.751 125.197) (width 0.7) (layer "F.Cu") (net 15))
 (segment (start 237.211 111.531) (end 237.211 125.451) (width 0.7) (layer "F.Cu") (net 16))
 (segment (start 237.211 125.451) (end 237.5 125.74) (width 0.7) (layer "F.Cu") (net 16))
 (segment (start 237.5 125.74) (end 237.5 128.26) (width 0.7) (layer "F.Cu") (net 16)))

